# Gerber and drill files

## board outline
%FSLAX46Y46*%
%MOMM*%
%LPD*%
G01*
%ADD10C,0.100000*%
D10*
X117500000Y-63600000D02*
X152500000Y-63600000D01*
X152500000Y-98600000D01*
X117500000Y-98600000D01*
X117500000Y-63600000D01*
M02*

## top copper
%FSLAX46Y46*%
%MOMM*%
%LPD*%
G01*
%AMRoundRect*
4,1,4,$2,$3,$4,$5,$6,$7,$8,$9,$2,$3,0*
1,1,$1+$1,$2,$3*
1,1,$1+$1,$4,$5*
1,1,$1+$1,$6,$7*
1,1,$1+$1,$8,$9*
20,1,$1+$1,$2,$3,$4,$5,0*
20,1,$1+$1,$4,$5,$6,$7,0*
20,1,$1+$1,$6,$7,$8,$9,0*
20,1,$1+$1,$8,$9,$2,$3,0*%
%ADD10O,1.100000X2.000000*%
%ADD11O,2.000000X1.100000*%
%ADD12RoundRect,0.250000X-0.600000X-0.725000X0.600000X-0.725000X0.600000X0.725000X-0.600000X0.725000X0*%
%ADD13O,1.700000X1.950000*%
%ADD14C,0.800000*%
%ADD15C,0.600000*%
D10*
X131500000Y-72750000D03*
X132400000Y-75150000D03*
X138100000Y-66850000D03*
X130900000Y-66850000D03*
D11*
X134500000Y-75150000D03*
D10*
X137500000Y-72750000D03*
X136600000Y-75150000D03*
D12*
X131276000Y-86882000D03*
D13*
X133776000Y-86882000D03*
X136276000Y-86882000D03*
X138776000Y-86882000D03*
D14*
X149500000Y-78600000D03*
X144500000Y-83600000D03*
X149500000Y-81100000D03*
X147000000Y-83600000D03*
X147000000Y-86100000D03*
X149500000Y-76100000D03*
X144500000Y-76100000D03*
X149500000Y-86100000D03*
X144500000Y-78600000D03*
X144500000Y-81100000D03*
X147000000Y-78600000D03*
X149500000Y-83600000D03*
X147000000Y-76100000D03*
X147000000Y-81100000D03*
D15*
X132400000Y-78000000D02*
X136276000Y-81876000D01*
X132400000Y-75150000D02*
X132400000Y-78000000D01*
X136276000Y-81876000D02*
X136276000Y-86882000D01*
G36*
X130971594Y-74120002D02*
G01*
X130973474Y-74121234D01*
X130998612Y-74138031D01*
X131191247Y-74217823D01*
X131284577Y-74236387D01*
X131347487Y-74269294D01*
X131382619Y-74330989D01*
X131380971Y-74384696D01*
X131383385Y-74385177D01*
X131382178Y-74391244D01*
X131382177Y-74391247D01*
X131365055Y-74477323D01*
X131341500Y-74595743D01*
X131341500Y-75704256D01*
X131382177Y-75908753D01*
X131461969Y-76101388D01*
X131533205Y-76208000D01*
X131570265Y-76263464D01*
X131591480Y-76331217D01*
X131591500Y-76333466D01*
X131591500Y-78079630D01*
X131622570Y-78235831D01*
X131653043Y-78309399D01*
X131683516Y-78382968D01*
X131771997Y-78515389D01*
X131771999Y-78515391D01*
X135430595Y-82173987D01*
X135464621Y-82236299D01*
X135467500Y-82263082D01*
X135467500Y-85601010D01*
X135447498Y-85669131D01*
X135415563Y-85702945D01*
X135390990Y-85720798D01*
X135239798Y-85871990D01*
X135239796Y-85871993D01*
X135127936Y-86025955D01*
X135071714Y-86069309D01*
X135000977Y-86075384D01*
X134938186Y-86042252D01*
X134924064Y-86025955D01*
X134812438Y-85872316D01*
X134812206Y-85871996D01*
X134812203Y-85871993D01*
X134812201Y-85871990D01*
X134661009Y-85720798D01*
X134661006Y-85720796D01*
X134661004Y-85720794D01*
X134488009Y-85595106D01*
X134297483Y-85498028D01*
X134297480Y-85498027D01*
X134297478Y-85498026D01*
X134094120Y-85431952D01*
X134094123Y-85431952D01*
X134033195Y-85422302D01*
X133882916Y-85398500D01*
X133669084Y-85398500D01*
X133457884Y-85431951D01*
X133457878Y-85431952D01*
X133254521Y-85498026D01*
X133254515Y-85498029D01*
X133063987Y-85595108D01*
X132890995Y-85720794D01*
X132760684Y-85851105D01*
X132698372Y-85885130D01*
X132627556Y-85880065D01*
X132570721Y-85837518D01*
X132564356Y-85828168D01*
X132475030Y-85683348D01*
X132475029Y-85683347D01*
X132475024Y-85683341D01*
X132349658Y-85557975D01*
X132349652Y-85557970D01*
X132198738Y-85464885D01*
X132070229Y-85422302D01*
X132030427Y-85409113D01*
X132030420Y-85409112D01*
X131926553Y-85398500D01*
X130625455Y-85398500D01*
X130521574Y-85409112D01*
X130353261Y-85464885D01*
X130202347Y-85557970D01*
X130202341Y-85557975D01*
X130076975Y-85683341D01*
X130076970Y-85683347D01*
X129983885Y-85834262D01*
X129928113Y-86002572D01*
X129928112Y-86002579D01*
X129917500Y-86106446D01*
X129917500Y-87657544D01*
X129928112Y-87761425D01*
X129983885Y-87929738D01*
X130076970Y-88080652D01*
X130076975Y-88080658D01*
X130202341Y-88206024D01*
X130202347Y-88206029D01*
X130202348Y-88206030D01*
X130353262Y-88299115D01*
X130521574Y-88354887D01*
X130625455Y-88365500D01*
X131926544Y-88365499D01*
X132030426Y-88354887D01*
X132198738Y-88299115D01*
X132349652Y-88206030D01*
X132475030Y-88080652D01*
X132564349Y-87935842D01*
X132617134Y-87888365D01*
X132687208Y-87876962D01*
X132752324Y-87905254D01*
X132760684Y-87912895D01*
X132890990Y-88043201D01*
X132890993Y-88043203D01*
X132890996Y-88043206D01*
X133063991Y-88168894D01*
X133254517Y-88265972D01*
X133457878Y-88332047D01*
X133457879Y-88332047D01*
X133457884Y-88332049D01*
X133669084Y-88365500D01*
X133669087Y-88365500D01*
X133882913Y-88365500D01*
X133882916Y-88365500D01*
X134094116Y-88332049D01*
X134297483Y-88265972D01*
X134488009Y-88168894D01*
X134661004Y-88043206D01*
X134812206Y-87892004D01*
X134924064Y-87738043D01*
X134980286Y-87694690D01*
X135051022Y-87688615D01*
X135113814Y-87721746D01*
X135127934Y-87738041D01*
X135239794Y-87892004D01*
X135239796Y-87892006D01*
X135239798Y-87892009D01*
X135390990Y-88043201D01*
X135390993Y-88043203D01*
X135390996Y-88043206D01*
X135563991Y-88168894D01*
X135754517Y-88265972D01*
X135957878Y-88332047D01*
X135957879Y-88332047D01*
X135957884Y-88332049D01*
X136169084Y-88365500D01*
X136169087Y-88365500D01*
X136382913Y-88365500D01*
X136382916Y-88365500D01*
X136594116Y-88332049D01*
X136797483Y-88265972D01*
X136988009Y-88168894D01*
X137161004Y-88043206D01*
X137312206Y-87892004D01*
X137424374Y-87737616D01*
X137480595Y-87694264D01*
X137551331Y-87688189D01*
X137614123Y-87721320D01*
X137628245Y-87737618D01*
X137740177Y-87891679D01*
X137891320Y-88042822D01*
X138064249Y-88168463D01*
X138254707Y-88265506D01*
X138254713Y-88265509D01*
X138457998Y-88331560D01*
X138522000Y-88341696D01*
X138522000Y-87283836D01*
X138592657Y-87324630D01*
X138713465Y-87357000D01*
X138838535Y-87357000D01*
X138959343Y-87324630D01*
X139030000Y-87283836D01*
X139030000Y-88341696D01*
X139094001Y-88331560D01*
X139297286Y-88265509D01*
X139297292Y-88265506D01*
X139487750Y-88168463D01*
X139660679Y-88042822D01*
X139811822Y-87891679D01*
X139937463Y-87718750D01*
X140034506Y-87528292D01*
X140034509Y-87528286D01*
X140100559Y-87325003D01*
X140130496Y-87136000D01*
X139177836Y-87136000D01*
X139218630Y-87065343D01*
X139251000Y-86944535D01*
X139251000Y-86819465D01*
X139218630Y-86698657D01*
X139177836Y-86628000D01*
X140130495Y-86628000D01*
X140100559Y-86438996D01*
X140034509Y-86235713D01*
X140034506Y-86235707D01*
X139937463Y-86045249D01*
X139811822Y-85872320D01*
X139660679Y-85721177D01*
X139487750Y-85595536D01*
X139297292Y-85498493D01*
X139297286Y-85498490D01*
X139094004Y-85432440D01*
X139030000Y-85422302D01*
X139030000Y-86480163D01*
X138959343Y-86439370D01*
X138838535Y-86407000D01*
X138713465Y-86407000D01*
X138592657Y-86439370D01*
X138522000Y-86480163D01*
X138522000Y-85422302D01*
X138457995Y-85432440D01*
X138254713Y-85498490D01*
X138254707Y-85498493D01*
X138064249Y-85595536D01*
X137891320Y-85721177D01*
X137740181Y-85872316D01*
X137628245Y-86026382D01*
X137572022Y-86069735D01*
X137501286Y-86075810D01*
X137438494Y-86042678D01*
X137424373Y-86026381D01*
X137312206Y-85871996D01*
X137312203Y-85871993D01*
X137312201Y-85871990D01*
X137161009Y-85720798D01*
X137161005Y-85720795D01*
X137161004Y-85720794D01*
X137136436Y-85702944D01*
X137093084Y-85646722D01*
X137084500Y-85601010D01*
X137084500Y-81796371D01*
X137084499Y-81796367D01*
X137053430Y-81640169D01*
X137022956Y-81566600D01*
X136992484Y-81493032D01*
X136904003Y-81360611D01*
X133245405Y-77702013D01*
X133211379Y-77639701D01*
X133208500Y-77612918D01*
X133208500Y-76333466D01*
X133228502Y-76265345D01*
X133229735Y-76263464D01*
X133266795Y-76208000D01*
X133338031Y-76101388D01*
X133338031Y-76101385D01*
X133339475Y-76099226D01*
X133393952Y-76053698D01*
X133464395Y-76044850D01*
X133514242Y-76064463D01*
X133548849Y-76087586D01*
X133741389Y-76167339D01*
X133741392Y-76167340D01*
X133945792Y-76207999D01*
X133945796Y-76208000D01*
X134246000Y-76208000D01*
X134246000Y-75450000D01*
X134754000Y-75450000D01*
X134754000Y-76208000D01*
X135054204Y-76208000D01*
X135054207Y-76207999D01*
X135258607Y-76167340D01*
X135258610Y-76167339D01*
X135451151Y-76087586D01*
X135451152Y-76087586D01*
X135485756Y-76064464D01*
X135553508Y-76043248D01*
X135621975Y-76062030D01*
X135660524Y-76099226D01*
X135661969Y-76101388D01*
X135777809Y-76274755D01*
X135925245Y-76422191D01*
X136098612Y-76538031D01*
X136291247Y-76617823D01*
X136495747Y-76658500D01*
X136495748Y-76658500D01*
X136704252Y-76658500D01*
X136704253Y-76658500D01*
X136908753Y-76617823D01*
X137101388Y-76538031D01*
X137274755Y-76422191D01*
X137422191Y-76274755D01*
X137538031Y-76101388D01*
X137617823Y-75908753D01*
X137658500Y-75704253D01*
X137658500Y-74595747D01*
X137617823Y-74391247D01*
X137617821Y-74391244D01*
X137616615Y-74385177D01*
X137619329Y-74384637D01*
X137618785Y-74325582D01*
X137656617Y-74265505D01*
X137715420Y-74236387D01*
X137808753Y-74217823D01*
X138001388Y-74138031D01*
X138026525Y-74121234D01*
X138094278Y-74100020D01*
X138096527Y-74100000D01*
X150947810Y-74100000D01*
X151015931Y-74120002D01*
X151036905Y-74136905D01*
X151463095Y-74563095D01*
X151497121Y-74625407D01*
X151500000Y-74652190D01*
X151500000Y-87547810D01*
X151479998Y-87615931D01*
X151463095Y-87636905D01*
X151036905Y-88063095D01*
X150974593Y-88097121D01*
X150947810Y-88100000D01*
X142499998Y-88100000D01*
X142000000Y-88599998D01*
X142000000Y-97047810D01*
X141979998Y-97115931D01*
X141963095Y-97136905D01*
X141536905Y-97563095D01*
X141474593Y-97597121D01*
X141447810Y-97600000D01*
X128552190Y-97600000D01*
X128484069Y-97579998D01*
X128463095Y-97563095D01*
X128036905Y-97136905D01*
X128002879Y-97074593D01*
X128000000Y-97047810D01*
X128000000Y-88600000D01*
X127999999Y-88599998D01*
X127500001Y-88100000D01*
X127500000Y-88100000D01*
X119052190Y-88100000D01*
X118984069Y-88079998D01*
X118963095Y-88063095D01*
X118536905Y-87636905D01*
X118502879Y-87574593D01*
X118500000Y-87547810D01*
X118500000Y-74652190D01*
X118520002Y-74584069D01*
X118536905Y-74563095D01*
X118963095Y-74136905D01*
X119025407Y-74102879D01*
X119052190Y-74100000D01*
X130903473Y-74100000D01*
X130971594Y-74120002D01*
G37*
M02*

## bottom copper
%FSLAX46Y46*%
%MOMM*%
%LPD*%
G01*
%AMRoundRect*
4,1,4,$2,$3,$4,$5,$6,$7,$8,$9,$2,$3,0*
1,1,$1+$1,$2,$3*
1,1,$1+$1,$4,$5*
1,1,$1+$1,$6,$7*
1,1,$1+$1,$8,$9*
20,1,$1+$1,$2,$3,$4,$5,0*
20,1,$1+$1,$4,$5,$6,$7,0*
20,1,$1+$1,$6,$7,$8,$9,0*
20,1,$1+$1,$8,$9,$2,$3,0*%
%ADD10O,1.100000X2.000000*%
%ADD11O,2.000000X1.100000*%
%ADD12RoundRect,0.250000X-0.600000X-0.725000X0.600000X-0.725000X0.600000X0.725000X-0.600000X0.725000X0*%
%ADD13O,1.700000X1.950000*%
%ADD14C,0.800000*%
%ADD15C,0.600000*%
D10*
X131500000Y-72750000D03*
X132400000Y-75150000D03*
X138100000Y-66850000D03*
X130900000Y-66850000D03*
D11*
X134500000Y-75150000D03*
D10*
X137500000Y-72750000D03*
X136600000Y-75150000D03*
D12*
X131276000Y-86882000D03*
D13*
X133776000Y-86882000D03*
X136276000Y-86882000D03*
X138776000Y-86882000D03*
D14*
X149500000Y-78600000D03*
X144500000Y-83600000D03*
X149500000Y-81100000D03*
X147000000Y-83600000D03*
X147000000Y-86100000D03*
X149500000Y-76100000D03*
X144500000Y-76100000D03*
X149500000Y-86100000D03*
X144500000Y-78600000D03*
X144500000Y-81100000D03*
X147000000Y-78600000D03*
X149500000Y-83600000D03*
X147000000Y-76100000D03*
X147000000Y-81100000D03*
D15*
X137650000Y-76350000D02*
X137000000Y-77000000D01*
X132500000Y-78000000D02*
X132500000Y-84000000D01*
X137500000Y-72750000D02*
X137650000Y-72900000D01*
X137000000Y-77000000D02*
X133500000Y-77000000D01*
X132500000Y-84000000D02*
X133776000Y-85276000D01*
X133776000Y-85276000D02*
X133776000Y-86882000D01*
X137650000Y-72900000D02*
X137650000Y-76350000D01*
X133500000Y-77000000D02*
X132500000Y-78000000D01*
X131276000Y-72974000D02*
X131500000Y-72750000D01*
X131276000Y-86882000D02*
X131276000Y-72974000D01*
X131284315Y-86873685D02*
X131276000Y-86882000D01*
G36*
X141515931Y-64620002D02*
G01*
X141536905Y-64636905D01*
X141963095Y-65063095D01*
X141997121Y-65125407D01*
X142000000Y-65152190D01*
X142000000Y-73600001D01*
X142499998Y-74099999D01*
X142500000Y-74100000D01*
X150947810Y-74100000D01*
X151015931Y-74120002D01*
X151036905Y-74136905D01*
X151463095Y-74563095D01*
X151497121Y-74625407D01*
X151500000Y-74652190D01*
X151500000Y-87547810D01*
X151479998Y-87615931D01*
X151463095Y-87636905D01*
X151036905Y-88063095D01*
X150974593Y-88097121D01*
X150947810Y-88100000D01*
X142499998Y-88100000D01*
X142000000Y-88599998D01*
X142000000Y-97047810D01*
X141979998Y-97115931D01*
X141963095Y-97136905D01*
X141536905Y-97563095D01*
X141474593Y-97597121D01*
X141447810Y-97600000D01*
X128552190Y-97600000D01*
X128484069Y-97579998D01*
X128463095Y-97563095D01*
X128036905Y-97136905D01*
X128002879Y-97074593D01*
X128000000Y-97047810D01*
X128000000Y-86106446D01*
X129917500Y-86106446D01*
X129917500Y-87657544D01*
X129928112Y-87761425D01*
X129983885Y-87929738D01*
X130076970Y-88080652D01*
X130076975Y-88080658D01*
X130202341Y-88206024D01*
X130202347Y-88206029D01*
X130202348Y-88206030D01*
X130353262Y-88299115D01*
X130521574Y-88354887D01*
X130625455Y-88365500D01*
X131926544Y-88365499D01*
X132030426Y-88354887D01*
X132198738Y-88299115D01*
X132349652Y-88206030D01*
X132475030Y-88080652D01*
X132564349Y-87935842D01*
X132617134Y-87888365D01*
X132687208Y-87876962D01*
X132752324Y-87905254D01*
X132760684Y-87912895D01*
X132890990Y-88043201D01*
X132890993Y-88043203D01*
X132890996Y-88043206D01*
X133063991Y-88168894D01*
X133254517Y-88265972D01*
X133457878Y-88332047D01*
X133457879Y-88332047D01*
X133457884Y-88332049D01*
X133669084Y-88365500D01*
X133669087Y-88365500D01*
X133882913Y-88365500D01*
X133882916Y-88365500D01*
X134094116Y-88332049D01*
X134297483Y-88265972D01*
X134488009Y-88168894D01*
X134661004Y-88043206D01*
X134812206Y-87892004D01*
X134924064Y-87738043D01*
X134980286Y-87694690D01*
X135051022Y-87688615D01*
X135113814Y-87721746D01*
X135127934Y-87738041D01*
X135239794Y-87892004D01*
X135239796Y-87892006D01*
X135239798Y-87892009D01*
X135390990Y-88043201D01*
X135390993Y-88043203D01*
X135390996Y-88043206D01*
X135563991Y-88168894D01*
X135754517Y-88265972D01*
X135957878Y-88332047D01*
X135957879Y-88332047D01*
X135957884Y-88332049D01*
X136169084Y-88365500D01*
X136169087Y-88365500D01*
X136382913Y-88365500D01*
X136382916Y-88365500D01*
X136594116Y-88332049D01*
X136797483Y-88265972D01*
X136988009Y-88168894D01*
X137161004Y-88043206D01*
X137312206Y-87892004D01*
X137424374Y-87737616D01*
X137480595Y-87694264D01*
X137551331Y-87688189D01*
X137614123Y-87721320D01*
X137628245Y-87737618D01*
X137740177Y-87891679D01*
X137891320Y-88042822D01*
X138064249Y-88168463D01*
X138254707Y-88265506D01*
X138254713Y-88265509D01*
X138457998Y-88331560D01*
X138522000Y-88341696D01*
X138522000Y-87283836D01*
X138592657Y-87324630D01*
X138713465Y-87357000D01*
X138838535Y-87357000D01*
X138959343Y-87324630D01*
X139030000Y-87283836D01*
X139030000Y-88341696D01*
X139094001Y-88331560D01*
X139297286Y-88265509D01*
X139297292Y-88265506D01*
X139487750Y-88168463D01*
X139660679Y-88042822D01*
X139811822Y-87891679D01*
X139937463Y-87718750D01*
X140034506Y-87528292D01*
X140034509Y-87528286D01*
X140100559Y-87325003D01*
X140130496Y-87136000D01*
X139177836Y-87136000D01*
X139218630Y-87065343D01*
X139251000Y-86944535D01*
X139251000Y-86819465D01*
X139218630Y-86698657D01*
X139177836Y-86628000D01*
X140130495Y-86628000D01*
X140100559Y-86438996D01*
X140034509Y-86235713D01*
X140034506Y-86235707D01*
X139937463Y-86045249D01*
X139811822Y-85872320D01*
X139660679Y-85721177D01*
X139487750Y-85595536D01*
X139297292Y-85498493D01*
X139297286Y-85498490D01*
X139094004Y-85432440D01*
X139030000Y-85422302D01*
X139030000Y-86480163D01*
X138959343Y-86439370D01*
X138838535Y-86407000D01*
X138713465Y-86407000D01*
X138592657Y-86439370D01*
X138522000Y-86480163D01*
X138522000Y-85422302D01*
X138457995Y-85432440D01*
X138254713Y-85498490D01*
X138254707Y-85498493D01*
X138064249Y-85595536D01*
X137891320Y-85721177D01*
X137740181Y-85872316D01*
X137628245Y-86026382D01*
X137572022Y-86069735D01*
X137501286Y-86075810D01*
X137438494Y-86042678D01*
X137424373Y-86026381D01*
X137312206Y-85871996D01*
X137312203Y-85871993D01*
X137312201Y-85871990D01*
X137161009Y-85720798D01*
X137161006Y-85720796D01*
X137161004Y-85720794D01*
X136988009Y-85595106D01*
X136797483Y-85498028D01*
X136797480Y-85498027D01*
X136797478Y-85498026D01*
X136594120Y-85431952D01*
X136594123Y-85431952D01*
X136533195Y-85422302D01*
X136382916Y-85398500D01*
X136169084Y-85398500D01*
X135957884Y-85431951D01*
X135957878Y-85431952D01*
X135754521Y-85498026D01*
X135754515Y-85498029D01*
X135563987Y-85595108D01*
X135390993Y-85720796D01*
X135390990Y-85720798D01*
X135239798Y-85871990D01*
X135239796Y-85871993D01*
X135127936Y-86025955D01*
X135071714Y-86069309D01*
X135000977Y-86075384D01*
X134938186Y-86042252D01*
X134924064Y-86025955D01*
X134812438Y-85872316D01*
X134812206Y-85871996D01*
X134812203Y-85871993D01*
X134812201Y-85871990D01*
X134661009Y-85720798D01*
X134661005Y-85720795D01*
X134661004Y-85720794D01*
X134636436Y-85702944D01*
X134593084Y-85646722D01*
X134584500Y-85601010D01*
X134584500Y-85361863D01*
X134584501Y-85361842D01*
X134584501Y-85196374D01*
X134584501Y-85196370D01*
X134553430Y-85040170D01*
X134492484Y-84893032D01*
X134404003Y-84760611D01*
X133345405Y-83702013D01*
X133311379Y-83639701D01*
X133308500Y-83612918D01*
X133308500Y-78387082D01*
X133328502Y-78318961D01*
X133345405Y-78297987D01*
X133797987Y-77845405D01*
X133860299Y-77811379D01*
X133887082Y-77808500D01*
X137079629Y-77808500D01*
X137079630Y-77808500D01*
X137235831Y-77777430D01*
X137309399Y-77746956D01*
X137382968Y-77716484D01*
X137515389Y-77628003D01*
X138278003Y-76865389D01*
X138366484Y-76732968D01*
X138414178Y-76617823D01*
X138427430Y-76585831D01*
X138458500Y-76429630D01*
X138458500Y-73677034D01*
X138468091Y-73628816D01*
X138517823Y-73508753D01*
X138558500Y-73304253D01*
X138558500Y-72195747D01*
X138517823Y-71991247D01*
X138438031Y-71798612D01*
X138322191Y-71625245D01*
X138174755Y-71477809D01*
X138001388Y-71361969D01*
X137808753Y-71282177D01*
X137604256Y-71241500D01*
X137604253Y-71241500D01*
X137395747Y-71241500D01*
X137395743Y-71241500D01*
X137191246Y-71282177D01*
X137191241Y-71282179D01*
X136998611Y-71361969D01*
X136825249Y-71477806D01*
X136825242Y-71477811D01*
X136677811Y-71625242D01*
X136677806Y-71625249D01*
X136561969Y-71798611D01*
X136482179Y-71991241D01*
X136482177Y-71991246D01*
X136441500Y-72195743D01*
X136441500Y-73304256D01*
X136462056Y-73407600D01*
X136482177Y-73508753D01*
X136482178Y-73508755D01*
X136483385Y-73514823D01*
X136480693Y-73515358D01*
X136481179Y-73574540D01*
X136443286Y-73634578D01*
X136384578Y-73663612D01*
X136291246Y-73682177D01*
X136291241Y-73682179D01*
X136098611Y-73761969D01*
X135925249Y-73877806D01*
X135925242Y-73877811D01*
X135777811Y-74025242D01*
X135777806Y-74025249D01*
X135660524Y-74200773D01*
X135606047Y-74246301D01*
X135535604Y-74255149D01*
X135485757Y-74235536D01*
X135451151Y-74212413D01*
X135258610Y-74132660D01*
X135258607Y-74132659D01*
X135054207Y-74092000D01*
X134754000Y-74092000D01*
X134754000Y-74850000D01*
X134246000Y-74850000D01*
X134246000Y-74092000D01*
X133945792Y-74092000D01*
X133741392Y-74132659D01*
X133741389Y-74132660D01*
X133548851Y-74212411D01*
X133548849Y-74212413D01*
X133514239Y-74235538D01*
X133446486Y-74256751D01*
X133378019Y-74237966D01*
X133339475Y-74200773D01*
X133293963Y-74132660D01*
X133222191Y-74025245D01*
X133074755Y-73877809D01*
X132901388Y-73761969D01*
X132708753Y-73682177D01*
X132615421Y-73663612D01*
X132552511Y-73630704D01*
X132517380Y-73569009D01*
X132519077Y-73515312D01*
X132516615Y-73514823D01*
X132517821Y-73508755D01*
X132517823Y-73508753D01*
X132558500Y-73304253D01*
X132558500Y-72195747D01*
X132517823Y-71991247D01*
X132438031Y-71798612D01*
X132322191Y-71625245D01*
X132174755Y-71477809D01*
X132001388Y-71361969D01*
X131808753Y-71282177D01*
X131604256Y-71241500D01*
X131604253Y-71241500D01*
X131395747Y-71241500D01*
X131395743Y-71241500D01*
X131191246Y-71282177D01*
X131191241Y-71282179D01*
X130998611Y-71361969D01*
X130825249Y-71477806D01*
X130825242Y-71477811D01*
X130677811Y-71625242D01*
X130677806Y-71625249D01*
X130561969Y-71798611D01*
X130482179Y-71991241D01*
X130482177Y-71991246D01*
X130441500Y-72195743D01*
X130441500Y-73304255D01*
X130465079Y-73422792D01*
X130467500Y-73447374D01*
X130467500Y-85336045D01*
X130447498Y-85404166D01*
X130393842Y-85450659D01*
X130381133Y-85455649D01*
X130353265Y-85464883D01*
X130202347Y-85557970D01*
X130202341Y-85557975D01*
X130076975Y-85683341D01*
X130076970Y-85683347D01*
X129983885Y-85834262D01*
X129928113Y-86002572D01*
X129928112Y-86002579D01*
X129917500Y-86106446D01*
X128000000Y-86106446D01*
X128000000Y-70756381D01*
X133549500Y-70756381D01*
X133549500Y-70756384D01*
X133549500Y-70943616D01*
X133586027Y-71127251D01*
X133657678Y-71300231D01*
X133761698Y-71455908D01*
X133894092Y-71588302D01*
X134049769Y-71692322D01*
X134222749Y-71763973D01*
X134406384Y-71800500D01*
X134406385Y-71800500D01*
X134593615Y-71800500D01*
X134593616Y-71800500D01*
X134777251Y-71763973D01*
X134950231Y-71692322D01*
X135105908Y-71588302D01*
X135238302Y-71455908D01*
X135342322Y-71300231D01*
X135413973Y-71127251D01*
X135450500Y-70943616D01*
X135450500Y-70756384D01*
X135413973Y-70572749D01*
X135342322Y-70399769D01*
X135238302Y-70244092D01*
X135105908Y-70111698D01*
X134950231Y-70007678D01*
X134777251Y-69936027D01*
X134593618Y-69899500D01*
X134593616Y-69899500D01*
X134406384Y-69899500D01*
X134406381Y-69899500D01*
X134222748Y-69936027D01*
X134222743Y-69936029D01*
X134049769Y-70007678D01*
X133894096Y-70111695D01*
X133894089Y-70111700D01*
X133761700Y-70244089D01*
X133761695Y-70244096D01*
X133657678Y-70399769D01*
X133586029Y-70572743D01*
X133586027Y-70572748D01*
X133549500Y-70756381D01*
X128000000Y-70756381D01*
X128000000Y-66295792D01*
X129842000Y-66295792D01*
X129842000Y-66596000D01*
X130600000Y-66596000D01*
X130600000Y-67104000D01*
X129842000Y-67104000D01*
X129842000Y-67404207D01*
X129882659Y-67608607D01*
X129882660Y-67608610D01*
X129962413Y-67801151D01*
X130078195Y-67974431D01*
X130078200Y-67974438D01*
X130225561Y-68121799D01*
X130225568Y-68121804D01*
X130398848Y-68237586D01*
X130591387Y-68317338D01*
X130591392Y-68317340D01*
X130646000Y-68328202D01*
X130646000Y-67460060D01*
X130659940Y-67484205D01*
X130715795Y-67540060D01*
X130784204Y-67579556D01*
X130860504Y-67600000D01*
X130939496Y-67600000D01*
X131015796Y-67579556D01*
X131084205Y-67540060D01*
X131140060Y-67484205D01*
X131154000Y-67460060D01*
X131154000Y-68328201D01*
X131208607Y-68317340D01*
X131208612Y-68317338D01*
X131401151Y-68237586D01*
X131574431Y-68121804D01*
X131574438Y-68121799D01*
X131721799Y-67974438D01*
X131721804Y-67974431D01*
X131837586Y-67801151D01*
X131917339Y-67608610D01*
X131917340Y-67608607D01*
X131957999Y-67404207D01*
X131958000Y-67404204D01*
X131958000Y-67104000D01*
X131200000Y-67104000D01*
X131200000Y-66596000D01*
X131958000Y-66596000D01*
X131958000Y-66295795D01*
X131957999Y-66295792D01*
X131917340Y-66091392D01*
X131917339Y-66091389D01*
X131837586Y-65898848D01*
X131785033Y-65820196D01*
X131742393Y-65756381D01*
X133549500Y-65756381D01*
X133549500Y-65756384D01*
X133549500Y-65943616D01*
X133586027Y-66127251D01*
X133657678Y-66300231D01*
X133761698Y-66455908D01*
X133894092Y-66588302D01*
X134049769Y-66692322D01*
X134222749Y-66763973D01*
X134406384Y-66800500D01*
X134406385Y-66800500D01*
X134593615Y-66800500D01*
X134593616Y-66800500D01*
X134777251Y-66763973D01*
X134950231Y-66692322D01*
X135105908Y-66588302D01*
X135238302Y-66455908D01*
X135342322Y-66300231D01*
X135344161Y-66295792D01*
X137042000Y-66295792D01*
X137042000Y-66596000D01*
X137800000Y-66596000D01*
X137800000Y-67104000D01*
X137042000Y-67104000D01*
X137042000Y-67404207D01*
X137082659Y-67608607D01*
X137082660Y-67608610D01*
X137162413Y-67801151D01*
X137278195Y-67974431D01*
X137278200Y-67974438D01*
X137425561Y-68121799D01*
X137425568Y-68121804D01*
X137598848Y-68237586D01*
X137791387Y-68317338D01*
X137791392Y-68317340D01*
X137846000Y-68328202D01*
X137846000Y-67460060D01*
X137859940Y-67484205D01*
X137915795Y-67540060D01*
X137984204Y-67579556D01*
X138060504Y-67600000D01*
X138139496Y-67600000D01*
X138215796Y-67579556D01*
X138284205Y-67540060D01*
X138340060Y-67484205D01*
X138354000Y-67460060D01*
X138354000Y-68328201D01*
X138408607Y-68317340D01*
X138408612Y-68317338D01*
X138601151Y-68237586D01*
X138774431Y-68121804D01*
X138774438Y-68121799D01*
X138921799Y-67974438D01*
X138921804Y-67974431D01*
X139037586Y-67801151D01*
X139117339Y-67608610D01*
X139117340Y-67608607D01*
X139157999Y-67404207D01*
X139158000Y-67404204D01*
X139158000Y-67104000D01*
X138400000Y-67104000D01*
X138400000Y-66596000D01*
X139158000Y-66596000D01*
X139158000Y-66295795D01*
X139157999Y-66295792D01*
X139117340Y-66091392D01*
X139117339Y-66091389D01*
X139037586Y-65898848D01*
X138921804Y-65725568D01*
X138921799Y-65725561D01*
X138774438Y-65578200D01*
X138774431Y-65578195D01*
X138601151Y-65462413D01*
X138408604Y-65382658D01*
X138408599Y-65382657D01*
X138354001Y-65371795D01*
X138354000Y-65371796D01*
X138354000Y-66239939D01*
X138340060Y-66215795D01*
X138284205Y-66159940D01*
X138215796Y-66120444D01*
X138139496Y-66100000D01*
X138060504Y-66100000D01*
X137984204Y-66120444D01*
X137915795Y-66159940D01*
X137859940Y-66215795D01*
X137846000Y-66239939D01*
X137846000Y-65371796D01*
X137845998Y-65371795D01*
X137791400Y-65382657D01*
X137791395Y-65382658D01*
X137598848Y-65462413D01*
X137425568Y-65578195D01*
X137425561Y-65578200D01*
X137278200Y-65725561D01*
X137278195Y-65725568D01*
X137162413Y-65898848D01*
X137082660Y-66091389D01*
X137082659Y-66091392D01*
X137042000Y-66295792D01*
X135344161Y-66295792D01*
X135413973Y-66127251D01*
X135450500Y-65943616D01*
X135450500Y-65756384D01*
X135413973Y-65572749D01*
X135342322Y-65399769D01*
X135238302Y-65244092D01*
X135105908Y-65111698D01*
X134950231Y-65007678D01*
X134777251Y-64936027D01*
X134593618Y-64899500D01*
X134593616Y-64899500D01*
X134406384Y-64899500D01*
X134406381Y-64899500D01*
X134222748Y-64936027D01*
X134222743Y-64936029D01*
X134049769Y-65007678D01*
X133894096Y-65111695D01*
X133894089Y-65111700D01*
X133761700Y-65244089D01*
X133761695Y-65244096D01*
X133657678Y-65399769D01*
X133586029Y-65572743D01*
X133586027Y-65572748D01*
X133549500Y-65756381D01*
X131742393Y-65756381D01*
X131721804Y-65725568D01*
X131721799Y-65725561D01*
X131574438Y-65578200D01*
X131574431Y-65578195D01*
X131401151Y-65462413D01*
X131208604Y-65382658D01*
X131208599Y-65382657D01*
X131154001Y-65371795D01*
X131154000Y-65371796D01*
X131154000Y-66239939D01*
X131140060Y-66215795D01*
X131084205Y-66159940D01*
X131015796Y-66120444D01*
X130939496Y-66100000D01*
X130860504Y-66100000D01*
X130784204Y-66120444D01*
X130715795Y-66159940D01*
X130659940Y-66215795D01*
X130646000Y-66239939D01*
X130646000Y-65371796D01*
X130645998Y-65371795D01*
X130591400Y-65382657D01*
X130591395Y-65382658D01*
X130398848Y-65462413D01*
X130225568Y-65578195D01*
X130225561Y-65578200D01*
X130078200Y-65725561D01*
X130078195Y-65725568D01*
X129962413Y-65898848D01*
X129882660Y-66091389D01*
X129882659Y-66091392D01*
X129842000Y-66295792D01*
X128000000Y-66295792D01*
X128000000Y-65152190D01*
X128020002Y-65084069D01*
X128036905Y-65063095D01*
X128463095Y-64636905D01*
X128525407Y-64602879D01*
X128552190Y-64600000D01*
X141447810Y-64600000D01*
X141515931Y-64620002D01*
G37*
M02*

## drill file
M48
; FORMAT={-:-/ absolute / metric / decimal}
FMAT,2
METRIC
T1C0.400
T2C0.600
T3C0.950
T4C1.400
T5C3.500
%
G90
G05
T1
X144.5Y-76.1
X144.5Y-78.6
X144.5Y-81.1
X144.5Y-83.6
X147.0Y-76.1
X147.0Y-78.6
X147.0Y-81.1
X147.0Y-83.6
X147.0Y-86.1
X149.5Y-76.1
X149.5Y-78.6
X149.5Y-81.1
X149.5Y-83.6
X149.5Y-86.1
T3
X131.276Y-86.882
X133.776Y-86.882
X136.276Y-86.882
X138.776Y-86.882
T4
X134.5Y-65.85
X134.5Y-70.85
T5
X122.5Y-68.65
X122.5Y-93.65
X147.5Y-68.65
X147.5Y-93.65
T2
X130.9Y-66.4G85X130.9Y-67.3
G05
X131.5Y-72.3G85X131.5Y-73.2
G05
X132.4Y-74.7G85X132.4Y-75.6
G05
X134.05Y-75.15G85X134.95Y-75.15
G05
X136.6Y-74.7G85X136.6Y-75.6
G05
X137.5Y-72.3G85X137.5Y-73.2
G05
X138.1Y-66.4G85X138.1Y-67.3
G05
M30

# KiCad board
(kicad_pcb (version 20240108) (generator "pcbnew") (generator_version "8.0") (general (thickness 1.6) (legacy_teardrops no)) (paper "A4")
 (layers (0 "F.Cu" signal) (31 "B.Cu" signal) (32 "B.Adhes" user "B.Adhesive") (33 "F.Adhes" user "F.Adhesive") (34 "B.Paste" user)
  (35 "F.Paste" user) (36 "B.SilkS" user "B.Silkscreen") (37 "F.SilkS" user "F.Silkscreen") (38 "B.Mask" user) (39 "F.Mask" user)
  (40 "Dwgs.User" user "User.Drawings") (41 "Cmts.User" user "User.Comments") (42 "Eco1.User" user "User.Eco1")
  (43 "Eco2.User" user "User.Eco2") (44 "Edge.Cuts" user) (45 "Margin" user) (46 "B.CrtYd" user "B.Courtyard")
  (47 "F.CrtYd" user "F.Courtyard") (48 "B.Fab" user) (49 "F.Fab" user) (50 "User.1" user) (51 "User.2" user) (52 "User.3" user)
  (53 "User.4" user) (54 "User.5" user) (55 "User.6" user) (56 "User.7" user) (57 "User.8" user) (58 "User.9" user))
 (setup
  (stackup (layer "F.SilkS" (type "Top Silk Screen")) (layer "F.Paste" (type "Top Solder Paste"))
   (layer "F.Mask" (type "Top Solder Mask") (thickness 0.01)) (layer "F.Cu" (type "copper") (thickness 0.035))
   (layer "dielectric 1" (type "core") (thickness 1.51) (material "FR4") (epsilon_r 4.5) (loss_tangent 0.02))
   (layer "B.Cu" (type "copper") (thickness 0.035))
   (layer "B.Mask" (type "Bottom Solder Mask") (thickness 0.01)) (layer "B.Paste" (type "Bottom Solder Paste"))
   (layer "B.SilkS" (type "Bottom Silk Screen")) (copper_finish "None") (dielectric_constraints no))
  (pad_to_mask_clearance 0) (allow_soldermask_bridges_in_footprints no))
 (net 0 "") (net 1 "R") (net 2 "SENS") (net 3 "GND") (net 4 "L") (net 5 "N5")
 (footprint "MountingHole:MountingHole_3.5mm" (layer "F.Cu") (at 147.5 68.65 180)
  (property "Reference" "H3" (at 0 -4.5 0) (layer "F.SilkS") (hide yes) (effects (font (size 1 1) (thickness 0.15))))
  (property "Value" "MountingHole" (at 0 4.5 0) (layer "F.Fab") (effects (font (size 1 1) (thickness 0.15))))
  (pad "" np_thru_hole circle (at 0 0 180) (size 3.5 3.5) (drill 3.5) (layers "*.Cu" "*.Mask")))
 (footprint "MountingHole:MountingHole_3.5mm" (layer "F.Cu") (at 122.5 93.65 180)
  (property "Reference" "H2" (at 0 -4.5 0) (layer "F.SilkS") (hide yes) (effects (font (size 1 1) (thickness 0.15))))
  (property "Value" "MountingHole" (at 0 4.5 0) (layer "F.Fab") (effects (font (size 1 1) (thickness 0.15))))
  (pad "" np_thru_hole circle (at 0 0 180) (size 3.5 3.5) (drill 3.5) (layers "*.Cu" "*.Mask")))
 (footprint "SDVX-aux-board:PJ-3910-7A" (layer "F.Cu") (at 134.5 71.1 -90)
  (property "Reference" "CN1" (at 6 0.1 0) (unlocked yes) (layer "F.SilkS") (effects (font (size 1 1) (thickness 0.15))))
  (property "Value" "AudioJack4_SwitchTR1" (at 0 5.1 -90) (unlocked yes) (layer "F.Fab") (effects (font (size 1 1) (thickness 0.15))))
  (pad "" np_thru_hole circle (at -5.25 0 270) (size 1.4 1.4) (drill 1.4) (layers "F&B.Cu"))
  (pad "" np_thru_hole circle (at -0.25 0 270) (size 1.4 1.4) (drill 1.4) (layers "F&B.Cu"))
  (pad "R1" thru_hole oval (at 1.65 3 270) (size 2 1.1) (drill oval 1.5 0.6) (layers "*.Cu" "*.Mask") (remove_unused_layers no) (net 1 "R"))
  (pad "R1N" thru_hole oval (at 4.05 2.1 270) (size 2 1.1) (drill oval 1.5 0.6) (layers "*.Cu" "*.Mask") (remove_unused_layers no)
   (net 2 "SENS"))
  (pad "R2" thru_hole oval (at -4.25 -3.6 270) (size 2 1.1) (drill oval 1.5 0.6) (layers "*.Cu" "*.Mask") (remove_unused_layers no)
   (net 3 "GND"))
  (pad "R2" thru_hole oval (at -4.25 3.6 270) (size 2 1.1) (drill oval 1.5 0.6) (layers "*.Cu" "*.Mask") (remove_unused_layers no)
   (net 3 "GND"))
  (pad "S" thru_hole oval (at 4.05 0) (size 2 1.1) (drill oval 1.5 0.6) (layers "*.Cu" "*.Mask") (remove_unused_layers no) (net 3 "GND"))
  (pad "T" thru_hole oval (at 1.65 -3 270) (size 2 1.1) (drill oval 1.5 0.6) (layers "*.Cu" "*.Mask") (remove_unused_layers no) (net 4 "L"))
  (pad "TN" thru_hole oval (at 4.05 -2.1 270) (size 2 1.1) (drill oval 1.5 0.6) (layers "*.Cu" "*.Mask") (remove_unused_layers no)
   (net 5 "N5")))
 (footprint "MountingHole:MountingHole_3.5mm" (layer "F.Cu") (at 122.5 68.65 180)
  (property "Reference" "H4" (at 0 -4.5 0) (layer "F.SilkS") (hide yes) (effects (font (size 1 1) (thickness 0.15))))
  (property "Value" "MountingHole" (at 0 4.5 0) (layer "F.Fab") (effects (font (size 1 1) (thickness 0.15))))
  (pad "" np_thru_hole circle (at 0 0 180) (size 3.5 3.5) (drill 3.5) (layers "*.Cu" "*.Mask")))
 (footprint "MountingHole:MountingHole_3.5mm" (layer "F.Cu") (at 147.5 93.65 180)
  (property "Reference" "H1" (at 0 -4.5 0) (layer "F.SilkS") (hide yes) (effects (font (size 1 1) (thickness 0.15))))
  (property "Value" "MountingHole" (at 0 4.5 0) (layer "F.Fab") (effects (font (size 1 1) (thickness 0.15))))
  (pad "" np_thru_hole circle (at 0 0 180) (size 3.5 3.5) (drill 3.5) (layers "*.Cu" "*.Mask")))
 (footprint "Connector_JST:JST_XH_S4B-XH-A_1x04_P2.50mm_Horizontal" (layer "F.Cu") (at 131.276 86.882)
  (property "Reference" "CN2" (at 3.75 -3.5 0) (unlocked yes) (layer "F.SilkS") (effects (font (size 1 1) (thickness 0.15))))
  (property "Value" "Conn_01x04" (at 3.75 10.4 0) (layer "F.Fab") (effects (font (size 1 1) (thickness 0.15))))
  (pad "1" thru_hole roundrect (at 0 0) (size 1.7 1.95) (drill 0.95) (layers "*.Cu" "*.Mask") (remove_unused_layers no)
   (roundrect_rratio 0.1470588235) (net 1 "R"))
  (pad "2" thru_hole oval (at 2.5 0) (size 1.7 1.95) (drill 0.95) (layers "*.Cu" "*.Mask") (remove_unused_layers no) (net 4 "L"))
  (pad "3" thru_hole oval (at 5 0) (size 1.7 1.95) (drill 0.95) (layers "*.Cu" "*.Mask") (remove_unused_layers no) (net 2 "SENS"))
  (pad "4" thru_hole oval (at 7.5 0) (size 1.7 1.95) (drill 0.95) (layers "*.Cu" "*.Mask") (remove_unused_layers no) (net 3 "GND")))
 (gr_rect (start 117.5 63.6) (end 152.5 98.6) (stroke (width 0.1) (type solid)) (fill none) (layer "Edge.Cuts"))
 (via (at 149.5 78.6) (size 0.8) (drill 0.4) (layers "F.Cu" "B.Cu") (free yes) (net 3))
 (via (at 144.5 83.6) (size 0.8) (drill 0.4) (layers "F.Cu" "B.Cu") (free yes) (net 3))
 (via (at 149.5 81.1) (size 0.8) (drill 0.4) (layers "F.Cu" "B.Cu") (free yes) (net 3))
 (via (at 147 83.6) (size 0.8) (drill 0.4) (layers "F.Cu" "B.Cu") (free yes) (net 3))
 (via (at 147 86.1) (size 0.8) (drill 0.4) (layers "F.Cu" "B.Cu") (free yes) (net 3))
 (via (at 149.5 76.1) (size 0.8) (drill 0.4) (layers "F.Cu" "B.Cu") (free yes) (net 3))
 (via (at 144.5 76.1) (size 0.8) (drill 0.4) (layers "F.Cu" "B.Cu") (free yes) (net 3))
 (via (at 149.5 86.1) (size 0.8) (drill 0.4) (layers "F.Cu" "B.Cu") (free yes) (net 3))
 (via (at 144.5 78.6) (size 0.8) (drill 0.4) (layers "F.Cu" "B.Cu") (free yes) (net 3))
 (via (at 144.5 81.1) (size 0.8) (drill 0.4) (layers "F.Cu" "B.Cu") (free yes) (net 3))
 (via (at 147 78.6) (size 0.8) (drill 0.4) (layers "F.Cu" "B.Cu") (free yes) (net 3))
 (via (at 149.5 83.6) (size 0.8) (drill 0.4) (layers "F.Cu" "B.Cu") (free yes) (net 3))
 (via (at 147 76.1) (size 0.8) (drill 0.4) (layers "F.Cu" "B.Cu") (free yes) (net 3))
 (via (at 147 81.1) (size 0.8) (drill 0.4) (layers "F.Cu" "B.Cu") (free yes) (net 3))
 (segment (start 137.65 76.35) (end 137 77) (width 0.6) (layer "B.Cu") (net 4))
 (segment (start 132.5 78) (end 132.5 84) (width 0.6) (layer "B.Cu") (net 4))
 (segment (start 137.5 72.75) (end 137.65 72.9) (width 0.6) (layer "B.Cu") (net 4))
 (segment (start 137 77) (end 133.5 77) (width 0.6) (layer "B.Cu") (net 4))
 (segment (start 132.5 84) (end 133.776 85.276) (width 0.6) (layer "B.Cu") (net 4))
 (segment (start 133.776 85.276) (end 133.776 86.882) (width 0.6) (layer "B.Cu") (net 4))
 (segment (start 137.65 72.9) (end 137.65 76.35) (width 0.6) (layer "B.Cu") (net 4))
 (segment (start 133.5 77) (end 132.5 78) (width 0.6) (layer "B.Cu") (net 4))
 (segment (start 132.4 78) (end 136.276 81.876) (width 0.6) (layer "F.Cu") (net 2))
 (segment (start 132.4 75.15) (end 132.4 78) (width 0.6) (layer "F.Cu") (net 2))
 (segment (start 136.276 81.876) (end 136.276 86.882) (width 0.6) (layer "F.Cu") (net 2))
 (segment (start 131.276 72.974) (end 131.5 72.75) (width 0.6) (layer "B.Cu") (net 1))
 (segment (start 131.276 86.882) (end 131.276 72.974) (width 0.6) (layer "B.Cu") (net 1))
 (segment (start 131.284315 86.873685) (end 131.276 86.882) (width 0.6) (layer "B.Cu") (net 1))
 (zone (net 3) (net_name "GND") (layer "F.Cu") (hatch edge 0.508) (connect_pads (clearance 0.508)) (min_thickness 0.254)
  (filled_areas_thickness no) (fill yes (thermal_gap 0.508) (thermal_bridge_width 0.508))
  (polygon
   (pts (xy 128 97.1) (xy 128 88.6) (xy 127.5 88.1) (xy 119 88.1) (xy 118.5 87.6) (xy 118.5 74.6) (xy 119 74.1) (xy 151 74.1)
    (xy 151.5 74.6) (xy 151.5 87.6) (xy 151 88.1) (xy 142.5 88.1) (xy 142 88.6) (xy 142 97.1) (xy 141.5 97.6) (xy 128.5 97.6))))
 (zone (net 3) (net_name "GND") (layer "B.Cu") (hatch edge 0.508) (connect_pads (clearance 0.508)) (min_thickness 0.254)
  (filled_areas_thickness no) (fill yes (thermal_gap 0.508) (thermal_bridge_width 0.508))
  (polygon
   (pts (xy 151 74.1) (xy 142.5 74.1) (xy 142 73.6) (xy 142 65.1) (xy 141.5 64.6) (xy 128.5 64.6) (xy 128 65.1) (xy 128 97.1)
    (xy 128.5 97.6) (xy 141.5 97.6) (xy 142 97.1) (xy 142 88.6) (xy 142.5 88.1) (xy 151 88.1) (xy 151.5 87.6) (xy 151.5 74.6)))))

